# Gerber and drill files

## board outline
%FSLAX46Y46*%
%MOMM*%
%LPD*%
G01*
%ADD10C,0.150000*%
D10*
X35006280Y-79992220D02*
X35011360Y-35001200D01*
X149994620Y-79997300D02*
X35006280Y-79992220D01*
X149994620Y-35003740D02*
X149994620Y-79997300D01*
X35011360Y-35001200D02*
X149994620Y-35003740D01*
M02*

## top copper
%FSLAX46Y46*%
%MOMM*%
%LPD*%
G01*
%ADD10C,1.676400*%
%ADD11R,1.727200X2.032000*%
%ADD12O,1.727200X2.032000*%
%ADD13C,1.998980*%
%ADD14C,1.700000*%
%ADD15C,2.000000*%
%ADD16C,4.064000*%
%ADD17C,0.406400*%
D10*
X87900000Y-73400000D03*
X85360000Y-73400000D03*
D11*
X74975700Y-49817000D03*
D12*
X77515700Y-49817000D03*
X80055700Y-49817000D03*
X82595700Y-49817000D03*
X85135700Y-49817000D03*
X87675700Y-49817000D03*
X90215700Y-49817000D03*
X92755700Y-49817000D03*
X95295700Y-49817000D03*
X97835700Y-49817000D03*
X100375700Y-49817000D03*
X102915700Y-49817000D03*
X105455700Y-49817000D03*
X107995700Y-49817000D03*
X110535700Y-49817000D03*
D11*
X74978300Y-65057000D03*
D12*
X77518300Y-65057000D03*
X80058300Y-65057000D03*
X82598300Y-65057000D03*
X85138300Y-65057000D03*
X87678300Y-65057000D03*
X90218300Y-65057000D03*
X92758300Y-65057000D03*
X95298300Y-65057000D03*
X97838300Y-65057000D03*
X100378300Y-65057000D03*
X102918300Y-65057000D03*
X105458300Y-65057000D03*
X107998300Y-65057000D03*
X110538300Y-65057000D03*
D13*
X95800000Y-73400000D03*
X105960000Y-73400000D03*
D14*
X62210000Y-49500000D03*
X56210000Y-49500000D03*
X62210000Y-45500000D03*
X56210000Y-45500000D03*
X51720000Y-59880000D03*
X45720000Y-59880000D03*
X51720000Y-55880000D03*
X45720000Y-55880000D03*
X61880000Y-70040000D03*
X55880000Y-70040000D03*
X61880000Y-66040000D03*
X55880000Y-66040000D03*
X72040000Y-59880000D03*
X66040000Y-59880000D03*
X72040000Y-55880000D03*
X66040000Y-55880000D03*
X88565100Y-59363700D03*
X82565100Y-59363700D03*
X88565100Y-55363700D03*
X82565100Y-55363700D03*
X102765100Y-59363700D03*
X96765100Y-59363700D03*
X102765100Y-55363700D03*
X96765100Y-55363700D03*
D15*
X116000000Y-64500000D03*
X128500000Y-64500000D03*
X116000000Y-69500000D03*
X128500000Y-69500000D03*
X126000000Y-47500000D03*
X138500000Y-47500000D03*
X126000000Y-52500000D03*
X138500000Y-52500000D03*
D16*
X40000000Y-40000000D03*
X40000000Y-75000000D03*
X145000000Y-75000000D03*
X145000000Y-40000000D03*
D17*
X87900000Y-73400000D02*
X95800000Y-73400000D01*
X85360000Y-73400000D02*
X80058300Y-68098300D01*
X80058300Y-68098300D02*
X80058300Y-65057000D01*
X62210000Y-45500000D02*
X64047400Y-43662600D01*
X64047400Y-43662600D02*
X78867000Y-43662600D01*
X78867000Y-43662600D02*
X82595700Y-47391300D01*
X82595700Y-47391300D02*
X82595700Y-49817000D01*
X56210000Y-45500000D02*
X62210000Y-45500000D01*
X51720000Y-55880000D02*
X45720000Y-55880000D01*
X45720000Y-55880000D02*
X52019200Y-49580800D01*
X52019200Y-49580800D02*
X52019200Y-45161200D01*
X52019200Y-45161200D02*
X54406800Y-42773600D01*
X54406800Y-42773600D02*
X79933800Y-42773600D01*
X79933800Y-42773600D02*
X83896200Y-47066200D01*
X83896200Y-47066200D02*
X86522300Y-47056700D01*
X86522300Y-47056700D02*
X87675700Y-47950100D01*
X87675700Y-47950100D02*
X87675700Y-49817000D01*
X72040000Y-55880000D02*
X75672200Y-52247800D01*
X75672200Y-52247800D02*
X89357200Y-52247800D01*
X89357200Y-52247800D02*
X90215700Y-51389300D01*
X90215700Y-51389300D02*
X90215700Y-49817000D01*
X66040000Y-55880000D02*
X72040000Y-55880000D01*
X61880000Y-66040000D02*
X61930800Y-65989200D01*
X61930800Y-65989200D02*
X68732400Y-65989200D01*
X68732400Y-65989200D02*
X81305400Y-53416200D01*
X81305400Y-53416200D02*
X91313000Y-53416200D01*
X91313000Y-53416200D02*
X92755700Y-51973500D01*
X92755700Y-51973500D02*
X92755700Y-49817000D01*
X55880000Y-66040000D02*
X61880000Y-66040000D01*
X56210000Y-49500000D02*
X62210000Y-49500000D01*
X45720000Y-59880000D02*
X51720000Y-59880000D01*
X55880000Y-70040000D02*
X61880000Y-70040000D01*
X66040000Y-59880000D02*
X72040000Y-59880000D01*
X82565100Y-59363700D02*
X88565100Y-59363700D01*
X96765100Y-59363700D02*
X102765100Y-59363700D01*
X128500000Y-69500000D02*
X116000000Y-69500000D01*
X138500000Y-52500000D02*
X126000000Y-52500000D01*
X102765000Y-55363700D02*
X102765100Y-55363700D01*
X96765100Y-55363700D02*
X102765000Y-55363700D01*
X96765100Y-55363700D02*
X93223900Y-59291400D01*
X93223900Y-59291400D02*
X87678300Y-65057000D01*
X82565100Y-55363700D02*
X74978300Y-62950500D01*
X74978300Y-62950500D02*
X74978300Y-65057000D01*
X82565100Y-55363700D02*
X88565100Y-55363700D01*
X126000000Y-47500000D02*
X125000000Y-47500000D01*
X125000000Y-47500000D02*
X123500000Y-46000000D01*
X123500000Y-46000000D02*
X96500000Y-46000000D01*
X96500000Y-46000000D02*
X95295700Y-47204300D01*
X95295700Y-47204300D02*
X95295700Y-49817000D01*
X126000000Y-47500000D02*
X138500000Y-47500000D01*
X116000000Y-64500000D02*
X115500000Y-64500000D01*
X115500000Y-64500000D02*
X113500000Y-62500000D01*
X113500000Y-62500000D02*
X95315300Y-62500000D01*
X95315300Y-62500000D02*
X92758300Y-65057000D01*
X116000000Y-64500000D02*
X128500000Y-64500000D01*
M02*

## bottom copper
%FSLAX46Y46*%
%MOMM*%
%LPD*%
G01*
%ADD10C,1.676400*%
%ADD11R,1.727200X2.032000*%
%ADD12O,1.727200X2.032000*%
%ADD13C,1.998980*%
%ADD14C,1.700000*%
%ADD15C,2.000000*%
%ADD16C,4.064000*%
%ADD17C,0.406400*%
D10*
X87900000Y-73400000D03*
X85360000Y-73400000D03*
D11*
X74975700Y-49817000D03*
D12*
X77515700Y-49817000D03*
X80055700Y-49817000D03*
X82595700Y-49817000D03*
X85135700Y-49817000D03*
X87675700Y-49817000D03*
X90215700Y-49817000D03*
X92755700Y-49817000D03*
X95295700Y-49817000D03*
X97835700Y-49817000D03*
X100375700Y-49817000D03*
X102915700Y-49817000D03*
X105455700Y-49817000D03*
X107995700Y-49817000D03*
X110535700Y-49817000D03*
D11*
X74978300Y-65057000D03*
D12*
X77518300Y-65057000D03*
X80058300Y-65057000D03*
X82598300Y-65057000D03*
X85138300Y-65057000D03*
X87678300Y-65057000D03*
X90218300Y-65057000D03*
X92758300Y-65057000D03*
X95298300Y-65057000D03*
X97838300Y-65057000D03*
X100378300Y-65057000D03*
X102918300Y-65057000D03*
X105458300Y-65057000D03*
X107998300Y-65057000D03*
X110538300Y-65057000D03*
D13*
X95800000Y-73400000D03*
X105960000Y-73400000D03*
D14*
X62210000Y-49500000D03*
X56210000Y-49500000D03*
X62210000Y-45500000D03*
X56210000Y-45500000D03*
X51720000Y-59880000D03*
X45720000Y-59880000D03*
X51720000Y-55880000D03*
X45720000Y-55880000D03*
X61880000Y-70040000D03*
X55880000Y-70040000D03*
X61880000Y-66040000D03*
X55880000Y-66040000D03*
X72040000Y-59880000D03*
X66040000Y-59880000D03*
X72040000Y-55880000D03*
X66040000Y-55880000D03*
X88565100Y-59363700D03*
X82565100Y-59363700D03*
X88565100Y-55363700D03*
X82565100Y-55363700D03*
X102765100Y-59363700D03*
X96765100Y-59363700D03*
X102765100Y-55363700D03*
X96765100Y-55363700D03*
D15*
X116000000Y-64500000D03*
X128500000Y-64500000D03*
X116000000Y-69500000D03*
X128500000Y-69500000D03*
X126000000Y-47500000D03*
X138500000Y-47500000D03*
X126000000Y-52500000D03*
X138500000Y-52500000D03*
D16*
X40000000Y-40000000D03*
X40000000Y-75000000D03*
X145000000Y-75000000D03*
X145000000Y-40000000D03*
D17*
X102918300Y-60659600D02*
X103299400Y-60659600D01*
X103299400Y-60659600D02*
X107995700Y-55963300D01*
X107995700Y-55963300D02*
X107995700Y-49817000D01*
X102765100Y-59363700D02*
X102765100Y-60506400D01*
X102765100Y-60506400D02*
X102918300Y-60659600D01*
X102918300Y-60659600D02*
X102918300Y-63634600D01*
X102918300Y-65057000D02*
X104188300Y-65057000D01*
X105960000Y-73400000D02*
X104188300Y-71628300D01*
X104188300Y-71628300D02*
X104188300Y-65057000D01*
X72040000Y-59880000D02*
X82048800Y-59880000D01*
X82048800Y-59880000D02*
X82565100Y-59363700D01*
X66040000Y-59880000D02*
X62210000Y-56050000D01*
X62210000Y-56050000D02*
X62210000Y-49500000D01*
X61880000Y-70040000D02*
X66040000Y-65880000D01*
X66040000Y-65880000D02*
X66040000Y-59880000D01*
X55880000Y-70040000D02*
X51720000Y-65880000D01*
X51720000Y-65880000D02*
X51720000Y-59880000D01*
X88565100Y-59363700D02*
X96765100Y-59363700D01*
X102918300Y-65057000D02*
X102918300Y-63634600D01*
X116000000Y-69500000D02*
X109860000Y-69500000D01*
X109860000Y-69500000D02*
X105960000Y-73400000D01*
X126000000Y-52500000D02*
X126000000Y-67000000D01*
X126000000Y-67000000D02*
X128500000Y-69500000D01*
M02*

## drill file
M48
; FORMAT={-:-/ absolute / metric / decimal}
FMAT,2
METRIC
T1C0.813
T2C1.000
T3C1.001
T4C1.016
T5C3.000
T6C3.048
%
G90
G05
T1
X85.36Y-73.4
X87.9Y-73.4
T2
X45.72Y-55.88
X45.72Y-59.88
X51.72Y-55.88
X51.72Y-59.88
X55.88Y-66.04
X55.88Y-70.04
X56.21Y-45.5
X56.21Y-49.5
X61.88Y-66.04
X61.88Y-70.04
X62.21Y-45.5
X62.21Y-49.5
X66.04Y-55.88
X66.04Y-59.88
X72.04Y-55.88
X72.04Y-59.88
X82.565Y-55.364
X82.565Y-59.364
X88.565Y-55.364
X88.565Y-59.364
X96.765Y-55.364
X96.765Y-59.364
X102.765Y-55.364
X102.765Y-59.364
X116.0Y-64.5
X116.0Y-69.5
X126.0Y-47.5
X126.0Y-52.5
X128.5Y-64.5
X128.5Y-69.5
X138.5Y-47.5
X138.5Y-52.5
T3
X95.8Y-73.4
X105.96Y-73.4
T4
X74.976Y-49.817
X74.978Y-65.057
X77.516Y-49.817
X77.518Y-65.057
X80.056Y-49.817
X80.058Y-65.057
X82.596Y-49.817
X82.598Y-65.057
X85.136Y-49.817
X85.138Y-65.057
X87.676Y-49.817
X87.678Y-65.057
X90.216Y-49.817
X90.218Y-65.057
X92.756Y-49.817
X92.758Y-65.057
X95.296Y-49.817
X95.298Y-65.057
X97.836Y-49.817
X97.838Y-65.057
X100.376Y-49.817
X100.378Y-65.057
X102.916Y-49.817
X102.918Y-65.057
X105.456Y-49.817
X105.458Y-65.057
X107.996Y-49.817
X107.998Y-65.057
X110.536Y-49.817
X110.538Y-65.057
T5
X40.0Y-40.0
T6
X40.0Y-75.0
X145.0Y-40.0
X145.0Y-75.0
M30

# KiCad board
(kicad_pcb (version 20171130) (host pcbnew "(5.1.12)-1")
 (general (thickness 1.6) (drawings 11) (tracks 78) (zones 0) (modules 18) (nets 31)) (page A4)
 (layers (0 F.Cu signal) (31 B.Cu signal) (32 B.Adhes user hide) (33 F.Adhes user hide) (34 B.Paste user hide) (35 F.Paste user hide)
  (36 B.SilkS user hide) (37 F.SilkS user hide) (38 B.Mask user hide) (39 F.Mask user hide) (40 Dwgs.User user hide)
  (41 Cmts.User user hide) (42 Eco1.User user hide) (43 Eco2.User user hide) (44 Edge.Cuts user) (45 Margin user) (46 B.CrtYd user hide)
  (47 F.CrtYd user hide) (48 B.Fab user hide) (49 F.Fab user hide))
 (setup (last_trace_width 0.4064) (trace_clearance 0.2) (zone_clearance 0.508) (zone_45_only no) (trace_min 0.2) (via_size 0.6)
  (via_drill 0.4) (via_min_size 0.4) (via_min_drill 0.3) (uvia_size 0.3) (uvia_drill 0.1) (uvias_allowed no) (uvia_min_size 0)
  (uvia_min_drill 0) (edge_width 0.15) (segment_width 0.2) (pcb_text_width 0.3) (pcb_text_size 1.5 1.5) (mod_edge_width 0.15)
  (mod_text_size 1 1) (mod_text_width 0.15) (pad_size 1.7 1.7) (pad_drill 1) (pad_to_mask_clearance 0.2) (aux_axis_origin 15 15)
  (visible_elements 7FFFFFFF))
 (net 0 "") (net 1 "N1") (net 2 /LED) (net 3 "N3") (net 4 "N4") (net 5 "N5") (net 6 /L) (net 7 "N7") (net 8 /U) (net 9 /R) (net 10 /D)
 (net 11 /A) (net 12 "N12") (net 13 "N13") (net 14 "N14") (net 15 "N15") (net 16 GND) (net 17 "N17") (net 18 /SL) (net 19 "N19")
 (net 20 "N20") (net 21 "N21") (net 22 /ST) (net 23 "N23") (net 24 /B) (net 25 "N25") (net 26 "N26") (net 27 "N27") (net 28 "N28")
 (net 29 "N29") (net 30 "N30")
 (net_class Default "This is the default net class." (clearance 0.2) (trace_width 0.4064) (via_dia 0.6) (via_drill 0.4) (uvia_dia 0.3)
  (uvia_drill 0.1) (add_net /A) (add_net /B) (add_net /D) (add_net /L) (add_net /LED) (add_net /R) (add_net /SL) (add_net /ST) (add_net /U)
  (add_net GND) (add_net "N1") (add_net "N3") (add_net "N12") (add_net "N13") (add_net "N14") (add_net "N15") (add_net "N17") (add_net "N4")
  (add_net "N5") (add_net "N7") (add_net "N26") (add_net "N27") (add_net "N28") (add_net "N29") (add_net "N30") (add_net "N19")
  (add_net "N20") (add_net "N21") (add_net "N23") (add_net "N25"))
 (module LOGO (layer B.Cu) (at 92.4306 44.6532)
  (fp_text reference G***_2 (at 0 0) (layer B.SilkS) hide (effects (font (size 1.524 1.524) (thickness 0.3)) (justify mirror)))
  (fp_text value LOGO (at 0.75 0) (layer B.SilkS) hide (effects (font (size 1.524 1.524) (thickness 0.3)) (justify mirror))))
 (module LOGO (layer F.Cu) (at 139.0396 63.246)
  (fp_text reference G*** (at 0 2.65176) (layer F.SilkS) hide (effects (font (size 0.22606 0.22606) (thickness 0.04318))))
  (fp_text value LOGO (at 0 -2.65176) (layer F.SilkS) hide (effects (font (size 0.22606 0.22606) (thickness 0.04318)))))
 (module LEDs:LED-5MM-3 (layer F.Cu) (at 87.9 73.4 180)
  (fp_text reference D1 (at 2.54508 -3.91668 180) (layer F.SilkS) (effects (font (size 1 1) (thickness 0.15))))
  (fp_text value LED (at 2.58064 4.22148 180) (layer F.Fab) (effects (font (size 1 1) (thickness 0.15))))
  (pad 1 thru_hole circle (at 0 0) (size 1.6764 1.6764) (drill 0.8128) (layers *.Cu *.Mask F.SilkS) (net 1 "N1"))
  (pad 2 thru_hole circle (at 2.54 0) (size 1.6764 1.6764) (drill 0.8128) (layers *.Cu *.Mask F.SilkS) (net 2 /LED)))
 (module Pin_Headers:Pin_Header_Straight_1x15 (layer B.Cu) (at 74.9757 49.817 270)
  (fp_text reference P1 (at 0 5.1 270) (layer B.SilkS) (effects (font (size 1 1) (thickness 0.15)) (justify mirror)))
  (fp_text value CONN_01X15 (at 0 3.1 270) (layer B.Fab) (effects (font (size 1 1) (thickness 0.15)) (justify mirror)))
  (pad 1 thru_hole rect (at 0 0 270) (size 2.032 1.7272) (drill 1.016) (layers *.Cu *.Mask B.SilkS) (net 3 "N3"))
  (pad 2 thru_hole oval (at 0 -2.54 270) (size 2.032 1.7272) (drill 1.016) (layers *.Cu *.Mask B.SilkS) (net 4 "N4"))
  (pad 3 thru_hole oval (at 0 -5.08 270) (size 2.032 1.7272) (drill 1.016) (layers *.Cu *.Mask B.SilkS) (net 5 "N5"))
  (pad 4 thru_hole oval (at 0 -7.62 270) (size 2.032 1.7272) (drill 1.016) (layers *.Cu *.Mask B.SilkS) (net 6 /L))
  (pad 5 thru_hole oval (at 0 -10.16 270) (size 2.032 1.7272) (drill 1.016) (layers *.Cu *.Mask B.SilkS) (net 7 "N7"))
  (pad 6 thru_hole oval (at 0 -12.7 270) (size 2.032 1.7272) (drill 1.016) (layers *.Cu *.Mask B.SilkS) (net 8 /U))
  (pad 7 thru_hole oval (at 0 -15.24 270) (size 2.032 1.7272) (drill 1.016) (layers *.Cu *.Mask B.SilkS) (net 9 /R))
  (pad 8 thru_hole oval (at 0 -17.78 270) (size 2.032 1.7272) (drill 1.016) (layers *.Cu *.Mask B.SilkS) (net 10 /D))
  (pad 9 thru_hole oval (at 0 -20.32 270) (size 2.032 1.7272) (drill 1.016) (layers *.Cu *.Mask B.SilkS) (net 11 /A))
  (pad 10 thru_hole oval (at 0 -22.86 270) (size 2.032 1.7272) (drill 1.016) (layers *.Cu *.Mask B.SilkS) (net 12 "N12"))
  (pad 11 thru_hole oval (at 0 -25.4 270) (size 2.032 1.7272) (drill 1.016) (layers *.Cu *.Mask B.SilkS) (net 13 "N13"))
  (pad 12 thru_hole oval (at 0 -27.94 270) (size 2.032 1.7272) (drill 1.016) (layers *.Cu *.Mask B.SilkS) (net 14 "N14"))
  (pad 13 thru_hole oval (at 0 -30.48 270) (size 2.032 1.7272) (drill 1.016) (layers *.Cu *.Mask B.SilkS) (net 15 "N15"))
  (pad 14 thru_hole oval (at 0 -33.02 270) (size 2.032 1.7272) (drill 1.016) (layers *.Cu *.Mask B.SilkS) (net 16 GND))
  (pad 15 thru_hole oval (at 0 -35.56 270) (size 2.032 1.7272) (drill 1.016) (layers *.Cu *.Mask B.SilkS) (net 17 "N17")))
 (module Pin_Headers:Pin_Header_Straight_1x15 (layer B.Cu) (at 74.9783 65.057 270)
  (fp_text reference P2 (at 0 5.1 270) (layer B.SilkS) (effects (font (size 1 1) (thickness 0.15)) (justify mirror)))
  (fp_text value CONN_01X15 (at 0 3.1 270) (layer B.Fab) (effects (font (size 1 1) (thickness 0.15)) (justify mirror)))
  (pad 1 thru_hole rect (at 0 0 270) (size 2.032 1.7272) (drill 1.016) (layers *.Cu *.Mask B.SilkS) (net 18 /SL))
  (pad 2 thru_hole oval (at 0 -2.54 270) (size 2.032 1.7272) (drill 1.016) (layers *.Cu *.Mask B.SilkS) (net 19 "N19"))
  (pad 3 thru_hole oval (at 0 -5.08 270) (size 2.032 1.7272) (drill 1.016) (layers *.Cu *.Mask B.SilkS) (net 2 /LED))
  (pad 4 thru_hole oval (at 0 -7.62 270) (size 2.032 1.7272) (drill 1.016) (layers *.Cu *.Mask B.SilkS) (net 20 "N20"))
  (pad 5 thru_hole oval (at 0 -10.16 270) (size 2.032 1.7272) (drill 1.016) (layers *.Cu *.Mask B.SilkS) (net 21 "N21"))
  (pad 6 thru_hole oval (at 0 -12.7 270) (size 2.032 1.7272) (drill 1.016) (layers *.Cu *.Mask B.SilkS) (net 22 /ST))
  (pad 7 thru_hole oval (at 0 -15.24 270) (size 2.032 1.7272) (drill 1.016) (layers *.Cu *.Mask B.SilkS) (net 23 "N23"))
  (pad 8 thru_hole oval (at 0 -17.78 270) (size 2.032 1.7272) (drill 1.016) (layers *.Cu *.Mask B.SilkS) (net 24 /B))
  (pad 9 thru_hole oval (at 0 -20.32 270) (size 2.032 1.7272) (drill 1.016) (layers *.Cu *.Mask B.SilkS) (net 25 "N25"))
  (pad 10 thru_hole oval (at 0 -22.86 270) (size 2.032 1.7272) (drill 1.016) (layers *.Cu *.Mask B.SilkS) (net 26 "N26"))
  (pad 11 thru_hole oval (at 0 -25.4 270) (size 2.032 1.7272) (drill 1.016) (layers *.Cu *.Mask B.SilkS) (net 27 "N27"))
  (pad 12 thru_hole oval (at 0 -27.94 270) (size 2.032 1.7272) (drill 1.016) (layers *.Cu *.Mask B.SilkS) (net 16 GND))
  (pad 13 thru_hole oval (at 0 -30.48 270) (size 2.032 1.7272) (drill 1.016) (layers *.Cu *.Mask B.SilkS) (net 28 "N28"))
  (pad 14 thru_hole oval (at 0 -33.02 270) (size 2.032 1.7272) (drill 1.016) (layers *.Cu *.Mask B.SilkS) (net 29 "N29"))
  (pad 15 thru_hole oval (at 0 -35.56 270) (size 2.032 1.7272) (drill 1.016) (layers *.Cu *.Mask B.SilkS) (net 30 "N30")))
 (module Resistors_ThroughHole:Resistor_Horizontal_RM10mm (layer F.Cu) (at 95.8 73.4)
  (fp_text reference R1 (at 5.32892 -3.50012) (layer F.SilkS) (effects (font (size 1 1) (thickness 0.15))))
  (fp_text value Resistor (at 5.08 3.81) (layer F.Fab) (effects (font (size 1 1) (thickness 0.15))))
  (pad 1 thru_hole circle (at 0 0) (size 1.99898 1.99898) (drill 1.00076) (layers *.Cu *.SilkS *.Mask) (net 1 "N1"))
  (pad 2 thru_hole circle (at 10.16 0) (size 1.99898 1.99898) (drill 1.00076) (layers *.Cu *.SilkS *.Mask) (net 16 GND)))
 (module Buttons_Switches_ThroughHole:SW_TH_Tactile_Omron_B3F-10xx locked (layer F.Cu) (at 56.21 45.5)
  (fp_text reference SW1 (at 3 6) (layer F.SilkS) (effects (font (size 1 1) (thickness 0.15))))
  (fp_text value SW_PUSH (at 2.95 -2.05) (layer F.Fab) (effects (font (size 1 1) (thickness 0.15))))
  (pad 4 thru_hole circle (at 6 4) (size 1.7 1.7) (drill 1) (layers *.Cu *.Mask) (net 16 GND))
  (pad 3 thru_hole circle (at 0 4) (size 1.7 1.7) (drill 1) (layers *.Cu *.Mask) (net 16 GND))
  (pad 1 thru_hole circle (at 6 0) (size 1.7 1.7) (drill 1) (layers *.Cu *.Mask) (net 6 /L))
  (pad 1 thru_hole circle (at 0 0) (size 1.7 1.7) (drill 1) (layers *.Cu *.Mask) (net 6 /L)))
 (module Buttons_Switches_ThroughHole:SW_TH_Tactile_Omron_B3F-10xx (layer F.Cu) (at 45.72 55.88)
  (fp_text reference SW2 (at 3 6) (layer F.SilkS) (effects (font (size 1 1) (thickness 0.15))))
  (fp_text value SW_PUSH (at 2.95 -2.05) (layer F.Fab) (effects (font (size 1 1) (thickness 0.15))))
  (pad 4 thru_hole circle (at 6 4) (size 1.7 1.7) (drill 1) (layers *.Cu *.Mask) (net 16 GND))
  (pad 3 thru_hole circle (at 0 4) (size 1.7 1.7) (drill 1) (layers *.Cu *.Mask) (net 16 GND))
  (pad 1 thru_hole circle (at 6 0) (size 1.7 1.7) (drill 1) (layers *.Cu *.Mask) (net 8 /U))
  (pad 1 thru_hole circle (at 0 0) (size 1.7 1.7) (drill 1) (layers *.Cu *.Mask) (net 8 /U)))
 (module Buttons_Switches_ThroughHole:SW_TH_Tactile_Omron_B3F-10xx (layer F.Cu) (at 55.88 66.04)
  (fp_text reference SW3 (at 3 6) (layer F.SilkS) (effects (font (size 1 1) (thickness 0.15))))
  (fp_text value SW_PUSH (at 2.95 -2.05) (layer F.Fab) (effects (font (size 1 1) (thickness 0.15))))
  (pad 4 thru_hole circle (at 6 4) (size 1.7 1.7) (drill 1) (layers *.Cu *.Mask) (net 16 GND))
  (pad 3 thru_hole circle (at 0 4) (size 1.7 1.7) (drill 1) (layers *.Cu *.Mask) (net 16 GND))
  (pad 2 thru_hole circle (at 6 0) (size 1.7 1.7) (drill 1) (layers *.Cu *.Mask) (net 10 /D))
  (pad 1 thru_hole circle (at 0 0) (size 1.7 1.7) (drill 1) (layers *.Cu *.Mask) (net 10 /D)))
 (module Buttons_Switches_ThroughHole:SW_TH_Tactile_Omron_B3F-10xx (layer F.Cu) (at 66.04 55.88)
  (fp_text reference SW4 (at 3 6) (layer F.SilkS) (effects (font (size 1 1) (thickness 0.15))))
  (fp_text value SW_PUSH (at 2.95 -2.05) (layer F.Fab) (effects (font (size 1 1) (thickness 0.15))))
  (pad 4 thru_hole circle (at 6 4) (size 1.7 1.7) (drill 1) (layers *.Cu *.Mask) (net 16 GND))
  (pad 3 thru_hole circle (at 0 4) (size 1.7 1.7) (drill 1) (layers *.Cu *.Mask) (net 16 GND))
  (pad 2 thru_hole circle (at 6 0) (size 1.7 1.7) (drill 1) (layers *.Cu *.Mask) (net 9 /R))
  (pad 1 thru_hole circle (at 0 0) (size 1.7 1.7) (drill 1) (layers *.Cu *.Mask) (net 9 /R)))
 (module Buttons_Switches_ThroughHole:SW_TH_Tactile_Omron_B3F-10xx (layer F.Cu) (at 82.5651 55.3637)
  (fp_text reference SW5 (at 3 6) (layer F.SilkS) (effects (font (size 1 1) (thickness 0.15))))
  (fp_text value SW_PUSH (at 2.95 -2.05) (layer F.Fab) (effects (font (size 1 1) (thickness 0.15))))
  (pad 4 thru_hole circle (at 6 4) (size 1.7 1.7) (drill 1) (layers *.Cu *.Mask) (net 16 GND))
  (pad 3 thru_hole circle (at 0 4) (size 1.7 1.7) (drill 1) (layers *.Cu *.Mask) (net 16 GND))
  (pad 2 thru_hole circle (at 6 0) (size 1.7 1.7) (drill 1) (layers *.Cu *.Mask) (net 18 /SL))
  (pad 1 thru_hole circle (at 0 0) (size 1.7 1.7) (drill 1) (layers *.Cu *.Mask) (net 18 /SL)))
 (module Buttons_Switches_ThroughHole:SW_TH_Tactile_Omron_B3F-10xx (layer F.Cu) (at 96.7651 55.3637)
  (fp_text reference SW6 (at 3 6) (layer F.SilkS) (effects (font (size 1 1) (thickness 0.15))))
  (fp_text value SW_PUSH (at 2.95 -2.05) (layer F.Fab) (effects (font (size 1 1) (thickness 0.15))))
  (pad 4 thru_hole circle (at 6 4) (size 1.7 1.7) (drill 1) (layers *.Cu *.Mask) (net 16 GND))
  (pad 3 thru_hole circle (at 0 4) (size 1.7 1.7) (drill 1) (layers *.Cu *.Mask) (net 16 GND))
  (pad 2 thru_hole circle (at 6 0) (size 1.7 1.7) (drill 1) (layers *.Cu *.Mask) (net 22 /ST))
  (pad 1 thru_hole circle (at 0 0) (size 1.7 1.7) (drill 1) (layers *.Cu *.Mask) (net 22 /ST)))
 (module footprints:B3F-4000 (layer F.Cu) (at 116 64.5)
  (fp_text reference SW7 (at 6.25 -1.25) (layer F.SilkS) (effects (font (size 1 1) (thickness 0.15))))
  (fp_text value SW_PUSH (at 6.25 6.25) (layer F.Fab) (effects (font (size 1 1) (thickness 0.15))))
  (pad 1 thru_hole circle (at 0 0) (size 2 2) (drill 1) (layers *.Cu *.Mask F.SilkS) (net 24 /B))
  (pad 1 thru_hole circle (at 12.5 0) (size 2 2) (drill 1) (layers *.Cu *.Mask F.SilkS) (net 24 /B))
  (pad 2 thru_hole circle (at 0 5) (size 2 2) (drill 1) (layers *.Cu *.Mask F.SilkS) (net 16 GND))
  (pad 2 thru_hole circle (at 12.5 5) (size 2 2) (drill 1) (layers *.Cu *.Mask F.SilkS) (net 16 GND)))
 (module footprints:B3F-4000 (layer F.Cu) (at 126 47.5)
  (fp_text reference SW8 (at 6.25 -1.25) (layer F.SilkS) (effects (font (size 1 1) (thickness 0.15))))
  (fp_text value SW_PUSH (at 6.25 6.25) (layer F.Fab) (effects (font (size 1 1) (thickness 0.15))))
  (pad 1 thru_hole circle (at 0 0) (size 2 2) (drill 1) (layers *.Cu *.Mask F.SilkS) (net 11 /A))
  (pad 1 thru_hole circle (at 12.5 0) (size 2 2) (drill 1) (layers *.Cu *.Mask F.SilkS) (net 11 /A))
  (pad 2 thru_hole circle (at 0 5) (size 2 2) (drill 1) (layers *.Cu *.Mask F.SilkS) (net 16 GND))
  (pad 2 thru_hole circle (at 12.5 5) (size 2 2) (drill 1) (layers *.Cu *.Mask F.SilkS) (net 16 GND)))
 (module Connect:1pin (layer F.Cu) (at 40 40)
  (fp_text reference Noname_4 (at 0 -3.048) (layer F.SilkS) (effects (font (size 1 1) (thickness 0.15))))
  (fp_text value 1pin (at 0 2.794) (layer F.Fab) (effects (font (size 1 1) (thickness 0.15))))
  (pad "" np_thru_hole circle (at 0 0) (size 4.064 4.064) (drill 3) (layers *.Cu *.Mask F.SilkS)))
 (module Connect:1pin (layer F.Cu) (at 40 75)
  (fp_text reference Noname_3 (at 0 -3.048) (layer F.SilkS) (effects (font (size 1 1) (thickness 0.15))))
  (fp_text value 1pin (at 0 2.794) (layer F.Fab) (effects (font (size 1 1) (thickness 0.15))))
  (pad "" np_thru_hole circle (at 0 0) (size 4.064 4.064) (drill 3.048) (layers *.Cu *.Mask F.SilkS)))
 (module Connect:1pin (layer F.Cu) (at 145 75)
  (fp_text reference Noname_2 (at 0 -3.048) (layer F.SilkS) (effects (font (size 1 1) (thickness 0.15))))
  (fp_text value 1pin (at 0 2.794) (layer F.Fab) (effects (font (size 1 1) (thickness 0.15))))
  (pad "" np_thru_hole circle (at 0 0) (size 4.064 4.064) (drill 3.048) (layers *.Cu *.Mask F.SilkS)))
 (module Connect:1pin (layer F.Cu) (at 145 40)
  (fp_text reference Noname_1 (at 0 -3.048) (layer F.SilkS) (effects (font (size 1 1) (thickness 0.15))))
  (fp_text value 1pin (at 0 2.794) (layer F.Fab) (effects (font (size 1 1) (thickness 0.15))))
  (pad "" np_thru_hole circle (at 0 0) (size 4.064 4.064) (drill 3.048) (layers *.Cu *.Mask F.SilkS)))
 (gr_line (start 35.00628 79.99222) (end 35.01136 35.0012) (layer Edge.Cuts) (width 0.15))
 (gr_line (start 149.99462 79.9973) (end 35.00628 79.99222) (layer Edge.Cuts) (width 0.15))
 (gr_line (start 149.99462 35.00374) (end 149.99462 79.9973) (layer Edge.Cuts) (width 0.15))
 (gr_line (start 35.01136 35.0012) (end 149.99462 35.00374) (layer Edge.Cuts) (width 0.15))
 (segment (start 87.9 73.4) (end 95.8 73.4) (width 0.4064) (layer F.Cu) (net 1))
 (segment (start 85.36 73.4) (end 80.0583 68.0983) (width 0.4064) (layer F.Cu) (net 2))
 (segment (start 80.0583 68.0983) (end 80.0583 65.057) (width 0.4064) (layer F.Cu) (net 2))
 (segment (start 62.21 45.5) (end 64.0474 43.6626) (width 0.4064) (layer F.Cu) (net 6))
 (segment (start 64.0474 43.6626) (end 78.867 43.6626) (width 0.4064) (layer F.Cu) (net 6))
 (segment (start 78.867 43.6626) (end 82.5957 47.3913) (width 0.4064) (layer F.Cu) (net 6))
 (segment (start 82.5957 47.3913) (end 82.5957 49.817) (width 0.4064) (layer F.Cu) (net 6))
 (segment (start 56.21 45.5) (end 62.21 45.5) (width 0.4064) (layer F.Cu) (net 6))
 (segment (start 51.72 55.88) (end 45.72 55.88) (width 0.4064) (layer F.Cu) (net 8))
 (segment (start 45.72 55.88) (end 52.0192 49.5808) (width 0.4064) (layer F.Cu) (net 8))
 (segment (start 52.0192 49.5808) (end 52.0192 45.1612) (width 0.4064) (layer F.Cu) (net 8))
 (segment (start 52.0192 45.1612) (end 54.4068 42.7736) (width 0.4064) (layer F.Cu) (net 8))
 (segment (start 54.4068 42.7736) (end 79.9338 42.7736) (width 0.4064) (layer F.Cu) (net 8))
 (segment (start 79.9338 42.7736) (end 83.8962 47.0662) (width 0.4064) (layer F.Cu) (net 8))
 (segment (start 83.8962 47.0662) (end 86.5223 47.0567) (width 0.4064) (layer F.Cu) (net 8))
 (segment (start 86.5223 47.0567) (end 87.6757 47.9501) (width 0.4064) (layer F.Cu) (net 8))
 (segment (start 87.6757 47.9501) (end 87.6757 49.817) (width 0.4064) (layer F.Cu) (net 8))
 (segment (start 72.04 55.88) (end 75.6722 52.2478) (width 0.4064) (layer F.Cu) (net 9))
 (segment (start 75.6722 52.2478) (end 89.3572 52.2478) (width 0.4064) (layer F.Cu) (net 9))
 (segment (start 89.3572 52.2478) (end 90.2157 51.3893) (width 0.4064) (layer F.Cu) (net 9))
 (segment (start 90.2157 51.3893) (end 90.2157 49.817) (width 0.4064) (layer F.Cu) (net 9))
 (segment (start 66.04 55.88) (end 72.04 55.88) (width 0.4064) (layer F.Cu) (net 9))
 (segment (start 61.88 66.04) (end 61.9308 65.9892) (width 0.4064) (layer F.Cu) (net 10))
 (segment (start 61.9308 65.9892) (end 68.7324 65.9892) (width 0.4064) (layer F.Cu) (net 10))
 (segment (start 68.7324 65.9892) (end 81.3054 53.4162) (width 0.4064) (layer F.Cu) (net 10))
 (segment (start 81.3054 53.4162) (end 91.313 53.4162) (width 0.4064) (layer F.Cu) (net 10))
 (segment (start 91.313 53.4162) (end 92.7557 51.9735) (width 0.4064) (layer F.Cu) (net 10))
 (segment (start 92.7557 51.9735) (end 92.7557 49.817) (width 0.4064) (layer F.Cu) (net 10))
 (segment (start 55.88 66.04) (end 61.88 66.04) (width 0.4064) (layer F.Cu) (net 10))
 (segment (start 102.9183 60.6596) (end 103.2994 60.6596) (width 0.4064) (layer B.Cu) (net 16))
 (segment (start 103.2994 60.6596) (end 107.9957 55.9633) (width 0.4064) (layer B.Cu) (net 16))
 (segment (start 107.9957 55.9633) (end 107.9957 49.817) (width 0.4064) (layer B.Cu) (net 16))
 (segment (start 102.7651 59.3637) (end 102.7651 60.5064) (width 0.4064) (layer B.Cu) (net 16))
 (segment (start 102.7651 60.5064) (end 102.9183 60.6596) (width 0.4064) (layer B.Cu) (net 16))
 (segment (start 102.9183 60.6596) (end 102.9183 63.6346) (width 0.4064) (layer B.Cu) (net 16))
 (segment (start 102.9183 65.057) (end 104.1883 65.057) (width 0.4064) (layer B.Cu) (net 16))
 (segment (start 105.96 73.4) (end 104.1883 71.6283) (width 0.4064) (layer B.Cu) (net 16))
 (segment (start 104.1883 71.6283) (end 104.1883 65.057) (width 0.4064) (layer B.Cu) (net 16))
 (segment (start 72.04 59.88) (end 82.0488 59.88) (width 0.4064) (layer B.Cu) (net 16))
 (segment (start 82.0488 59.88) (end 82.5651 59.3637) (width 0.4064) (layer B.Cu) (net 16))
 (segment (start 56.21 49.5) (end 62.21 49.5) (width 0.4064) (layer F.Cu) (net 16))
 (segment (start 66.04 59.88) (end 62.21 56.05) (width 0.4064) (layer B.Cu) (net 16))
 (segment (start 62.21 56.05) (end 62.21 49.5) (width 0.4064) (layer B.Cu) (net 16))
 (segment (start 61.88 70.04) (end 66.04 65.88) (width 0.4064) (layer B.Cu) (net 16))
 (segment (start 66.04 65.88) (end 66.04 59.88) (width 0.4064) (layer B.Cu) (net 16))
 (segment (start 45.72 59.88) (end 51.72 59.88) (width 0.4064) (layer F.Cu) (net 16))
 (segment (start 55.88 70.04) (end 51.72 65.88) (width 0.4064) (layer B.Cu) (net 16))
 (segment (start 51.72 65.88) (end 51.72 59.88) (width 0.4064) (layer B.Cu) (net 16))
 (segment (start 55.88 70.04) (end 61.88 70.04) (width 0.4064) (layer F.Cu) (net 16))
 (segment (start 66.04 59.88) (end 72.04 59.88) (width 0.4064) (layer F.Cu) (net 16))
 (segment (start 88.5651 59.3637) (end 96.7651 59.3637) (width 0.4064) (layer B.Cu) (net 16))
 (segment (start 82.5651 59.3637) (end 88.5651 59.3637) (width 0.4064) (layer F.Cu) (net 16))
 (segment (start 102.9183 65.057) (end 102.9183 63.6346) (width 0.4064) (layer B.Cu) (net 16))
 (segment (start 96.7651 59.3637) (end 102.7651 59.3637) (width 0.4064) (layer F.Cu) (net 16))
 (segment (start 116 69.5) (end 109.86 69.5) (width 0.4064) (layer B.Cu) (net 16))
 (segment (start 109.86 69.5) (end 105.96 73.4) (width 0.4064) (layer B.Cu) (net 16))
 (segment (start 128.5 69.5) (end 116 69.5) (width 0.4064) (layer F.Cu) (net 16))
 (segment (start 126 52.5) (end 126 67) (width 0.4064) (layer B.Cu) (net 16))
 (segment (start 126 67) (end 128.5 69.5) (width 0.4064) (layer B.Cu) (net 16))
 (segment (start 138.5 52.5) (end 126 52.5) (width 0.4064) (layer F.Cu) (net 16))
 (segment (start 102.765 55.3637) (end 102.7651 55.3637) (width 0.4064) (layer F.Cu) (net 22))
 (segment (start 96.7651 55.3637) (end 102.765 55.3637) (width 0.4064) (layer F.Cu) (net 22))
 (segment (start 96.7651 55.3637) (end 93.2239 59.2914) (width 0.4064) (layer F.Cu) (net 22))
 (segment (start 93.2239 59.2914) (end 87.6783 65.057) (width 0.4064) (layer F.Cu) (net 22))
 (segment (start 82.5651 55.3637) (end 74.9783 62.9505) (width 0.4064) (layer F.Cu) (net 18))
 (segment (start 74.9783 62.9505) (end 74.9783 65.057) (width 0.4064) (layer F.Cu) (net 18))
 (segment (start 82.5651 55.3637) (end 88.5651 55.3637) (width 0.4064) (layer F.Cu) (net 18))
 (segment (start 126 47.5) (end 125 47.5) (width 0.4064) (layer F.Cu) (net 11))
 (segment (start 125 47.5) (end 123.5 46) (width 0.4064) (layer F.Cu) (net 11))
 (segment (start 123.5 46) (end 96.5 46) (width 0.4064) (layer F.Cu) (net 11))
 (segment (start 96.5 46) (end 95.2957 47.2043) (width 0.4064) (layer F.Cu) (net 11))
 (segment (start 95.2957 47.2043) (end 95.2957 49.817) (width 0.4064) (layer F.Cu) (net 11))
 (segment (start 126 47.5) (end 138.5 47.5) (width 0.4064) (layer F.Cu) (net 11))
 (segment (start 116 64.5) (end 115.5 64.5) (width 0.4064) (layer F.Cu) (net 24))
 (segment (start 115.5 64.5) (end 113.5 62.5) (width 0.4064) (layer F.Cu) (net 24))
 (segment (start 113.5 62.5) (end 95.3153 62.5) (width 0.4064) (layer F.Cu) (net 24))
 (segment (start 95.3153 62.5) (end 92.7583 65.057) (width 0.4064) (layer F.Cu) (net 24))
 (segment (start 116 64.5) (end 128.5 64.5) (width 0.4064) (layer F.Cu) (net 24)))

